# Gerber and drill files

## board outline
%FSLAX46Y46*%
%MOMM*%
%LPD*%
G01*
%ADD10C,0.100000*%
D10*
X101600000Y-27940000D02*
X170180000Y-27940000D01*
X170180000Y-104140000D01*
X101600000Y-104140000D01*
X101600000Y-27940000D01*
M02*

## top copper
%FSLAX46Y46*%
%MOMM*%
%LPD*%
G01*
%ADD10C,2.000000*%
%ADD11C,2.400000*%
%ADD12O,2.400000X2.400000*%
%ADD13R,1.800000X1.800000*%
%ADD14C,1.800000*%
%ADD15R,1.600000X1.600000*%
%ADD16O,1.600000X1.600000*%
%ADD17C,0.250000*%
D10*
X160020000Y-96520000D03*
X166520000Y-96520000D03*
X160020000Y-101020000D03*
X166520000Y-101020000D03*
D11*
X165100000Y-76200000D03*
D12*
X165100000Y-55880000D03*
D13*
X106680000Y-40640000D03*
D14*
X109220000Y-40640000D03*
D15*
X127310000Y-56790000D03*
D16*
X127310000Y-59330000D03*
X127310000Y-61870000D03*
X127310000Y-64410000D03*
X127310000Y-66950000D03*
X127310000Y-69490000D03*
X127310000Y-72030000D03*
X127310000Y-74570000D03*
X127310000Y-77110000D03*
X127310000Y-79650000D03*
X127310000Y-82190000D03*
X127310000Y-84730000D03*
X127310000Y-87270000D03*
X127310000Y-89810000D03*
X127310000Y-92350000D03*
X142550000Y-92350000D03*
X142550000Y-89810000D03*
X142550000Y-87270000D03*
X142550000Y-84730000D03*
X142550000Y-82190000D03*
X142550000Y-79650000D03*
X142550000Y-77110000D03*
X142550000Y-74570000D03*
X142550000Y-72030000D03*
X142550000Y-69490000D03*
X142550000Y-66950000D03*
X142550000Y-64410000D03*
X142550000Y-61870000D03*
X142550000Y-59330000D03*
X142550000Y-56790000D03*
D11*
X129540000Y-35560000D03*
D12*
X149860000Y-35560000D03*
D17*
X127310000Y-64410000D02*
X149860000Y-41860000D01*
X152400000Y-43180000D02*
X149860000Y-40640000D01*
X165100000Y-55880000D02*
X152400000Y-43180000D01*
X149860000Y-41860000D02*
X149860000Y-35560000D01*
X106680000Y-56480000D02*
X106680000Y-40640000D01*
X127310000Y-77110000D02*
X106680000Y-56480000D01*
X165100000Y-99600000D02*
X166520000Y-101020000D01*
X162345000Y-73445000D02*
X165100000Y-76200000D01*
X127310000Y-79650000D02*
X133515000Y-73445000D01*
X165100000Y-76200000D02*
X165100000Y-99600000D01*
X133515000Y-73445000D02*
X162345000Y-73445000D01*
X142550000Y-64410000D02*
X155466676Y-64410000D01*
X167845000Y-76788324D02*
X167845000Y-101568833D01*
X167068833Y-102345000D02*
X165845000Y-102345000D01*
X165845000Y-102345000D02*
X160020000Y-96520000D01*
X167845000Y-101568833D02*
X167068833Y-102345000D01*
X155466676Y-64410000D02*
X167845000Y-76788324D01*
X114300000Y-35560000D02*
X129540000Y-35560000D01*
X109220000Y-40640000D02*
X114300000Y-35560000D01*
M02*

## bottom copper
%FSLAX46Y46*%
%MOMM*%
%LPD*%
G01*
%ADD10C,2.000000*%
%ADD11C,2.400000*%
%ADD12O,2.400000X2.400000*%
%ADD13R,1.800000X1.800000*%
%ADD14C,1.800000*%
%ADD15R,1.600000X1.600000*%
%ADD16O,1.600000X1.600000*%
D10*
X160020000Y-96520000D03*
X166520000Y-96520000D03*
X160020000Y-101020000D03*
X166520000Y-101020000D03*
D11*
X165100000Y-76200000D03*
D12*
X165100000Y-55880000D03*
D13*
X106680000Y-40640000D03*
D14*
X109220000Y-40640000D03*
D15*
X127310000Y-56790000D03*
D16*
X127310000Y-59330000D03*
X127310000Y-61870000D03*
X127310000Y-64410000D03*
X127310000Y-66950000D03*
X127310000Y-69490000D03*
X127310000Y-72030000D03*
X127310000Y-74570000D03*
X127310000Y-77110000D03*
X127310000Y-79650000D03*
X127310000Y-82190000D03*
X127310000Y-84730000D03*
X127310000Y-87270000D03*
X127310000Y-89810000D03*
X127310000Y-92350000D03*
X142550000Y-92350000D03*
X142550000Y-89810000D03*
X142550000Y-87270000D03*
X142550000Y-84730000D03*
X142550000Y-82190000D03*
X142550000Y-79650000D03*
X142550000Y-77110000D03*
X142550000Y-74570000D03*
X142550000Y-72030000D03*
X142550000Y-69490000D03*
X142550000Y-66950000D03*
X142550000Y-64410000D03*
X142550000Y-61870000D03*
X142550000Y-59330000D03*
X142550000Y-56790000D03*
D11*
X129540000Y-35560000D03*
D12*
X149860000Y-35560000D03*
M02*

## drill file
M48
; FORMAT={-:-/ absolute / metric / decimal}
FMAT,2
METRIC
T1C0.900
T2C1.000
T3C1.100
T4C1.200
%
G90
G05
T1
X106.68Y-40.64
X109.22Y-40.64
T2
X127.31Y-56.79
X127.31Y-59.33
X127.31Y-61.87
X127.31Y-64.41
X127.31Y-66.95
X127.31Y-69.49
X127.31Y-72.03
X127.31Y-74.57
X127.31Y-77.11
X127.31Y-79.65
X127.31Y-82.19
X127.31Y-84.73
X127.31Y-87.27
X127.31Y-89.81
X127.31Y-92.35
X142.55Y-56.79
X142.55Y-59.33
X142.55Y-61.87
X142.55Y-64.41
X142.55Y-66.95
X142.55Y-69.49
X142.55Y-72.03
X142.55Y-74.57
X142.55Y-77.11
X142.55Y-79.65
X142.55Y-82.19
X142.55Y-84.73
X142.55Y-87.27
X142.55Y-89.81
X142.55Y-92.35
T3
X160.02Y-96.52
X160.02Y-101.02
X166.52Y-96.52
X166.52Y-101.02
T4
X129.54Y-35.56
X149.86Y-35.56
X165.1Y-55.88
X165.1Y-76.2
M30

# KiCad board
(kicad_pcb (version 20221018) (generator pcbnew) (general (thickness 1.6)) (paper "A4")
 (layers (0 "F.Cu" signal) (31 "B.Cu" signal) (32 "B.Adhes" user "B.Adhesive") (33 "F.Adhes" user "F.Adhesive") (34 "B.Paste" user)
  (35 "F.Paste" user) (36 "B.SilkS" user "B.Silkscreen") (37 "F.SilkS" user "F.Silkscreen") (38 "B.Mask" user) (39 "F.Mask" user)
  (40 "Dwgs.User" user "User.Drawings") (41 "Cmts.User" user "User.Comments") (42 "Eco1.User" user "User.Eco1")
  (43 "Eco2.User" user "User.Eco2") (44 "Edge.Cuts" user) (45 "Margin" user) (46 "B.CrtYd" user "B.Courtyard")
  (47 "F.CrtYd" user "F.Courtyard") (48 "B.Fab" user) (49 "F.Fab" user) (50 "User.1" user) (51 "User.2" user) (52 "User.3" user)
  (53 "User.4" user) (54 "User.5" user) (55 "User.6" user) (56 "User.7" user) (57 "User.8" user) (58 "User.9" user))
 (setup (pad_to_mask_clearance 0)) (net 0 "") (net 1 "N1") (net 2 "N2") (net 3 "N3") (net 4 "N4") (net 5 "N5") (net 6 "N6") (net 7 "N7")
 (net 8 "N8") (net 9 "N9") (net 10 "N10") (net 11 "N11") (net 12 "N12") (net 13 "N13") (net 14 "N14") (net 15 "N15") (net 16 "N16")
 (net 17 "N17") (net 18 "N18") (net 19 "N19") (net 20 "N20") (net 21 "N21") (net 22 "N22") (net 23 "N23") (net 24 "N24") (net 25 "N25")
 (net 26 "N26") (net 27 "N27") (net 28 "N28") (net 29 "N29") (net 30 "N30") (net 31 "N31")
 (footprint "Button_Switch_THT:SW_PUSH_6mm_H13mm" (layer "F.Cu") (at 160.02 96.52)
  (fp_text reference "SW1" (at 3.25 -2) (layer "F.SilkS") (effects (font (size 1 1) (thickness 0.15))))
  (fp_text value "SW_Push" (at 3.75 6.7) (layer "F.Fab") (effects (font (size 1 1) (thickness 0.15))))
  (pad "1" thru_hole circle (at 0 0 90) (size 2 2) (drill 1.1) (layers "*.Cu" "*.Mask") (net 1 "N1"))
  (pad "1" thru_hole circle (at 6.5 0 90) (size 2 2) (drill 1.1) (layers "*.Cu" "*.Mask") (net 1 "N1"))
  (pad "2" thru_hole circle (at 0 4.5 90) (size 2 2) (drill 1.1) (layers "*.Cu" "*.Mask") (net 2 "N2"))
  (pad "2" thru_hole circle (at 6.5 4.5 90) (size 2 2) (drill 1.1) (layers "*.Cu" "*.Mask") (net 2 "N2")))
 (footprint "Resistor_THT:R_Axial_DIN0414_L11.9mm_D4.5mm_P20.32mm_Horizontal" (layer "F.Cu") (at 165.1 76.2 90)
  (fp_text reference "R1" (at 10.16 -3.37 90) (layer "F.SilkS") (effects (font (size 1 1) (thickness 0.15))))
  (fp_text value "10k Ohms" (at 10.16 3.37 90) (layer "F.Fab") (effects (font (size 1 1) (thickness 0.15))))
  (pad "1" thru_hole circle (at 0 0 90) (size 2.4 2.4) (drill 1.2) (layers "*.Cu" "*.Mask") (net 2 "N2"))
  (pad "2" thru_hole oval (at 20.32 0 90) (size 2.4 2.4) (drill 1.2) (layers "*.Cu" "*.Mask") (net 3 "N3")))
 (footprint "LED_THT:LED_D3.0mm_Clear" (layer "F.Cu") (at 106.68 40.64)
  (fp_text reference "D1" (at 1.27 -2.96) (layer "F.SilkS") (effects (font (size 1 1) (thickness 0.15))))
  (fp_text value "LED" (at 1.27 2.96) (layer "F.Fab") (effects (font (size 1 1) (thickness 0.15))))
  (pad "1" thru_hole rect (at 0 0) (size 1.8 1.8) (drill 0.9) (layers "*.Cu" "*.Mask") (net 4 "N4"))
  (pad "2" thru_hole circle (at 2.54 0) (size 1.8 1.8) (drill 0.9) (layers "*.Cu" "*.Mask") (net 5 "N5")))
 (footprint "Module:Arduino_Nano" (layer "F.Cu") (at 127.31 56.79)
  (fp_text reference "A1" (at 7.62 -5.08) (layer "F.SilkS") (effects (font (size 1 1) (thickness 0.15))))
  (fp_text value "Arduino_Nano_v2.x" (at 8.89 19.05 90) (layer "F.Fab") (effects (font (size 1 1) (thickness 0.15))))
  (pad "1" thru_hole rect (at 0 0) (size 1.6 1.6) (drill 1) (layers "*.Cu" "*.Mask") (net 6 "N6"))
  (pad "2" thru_hole oval (at 0 2.54) (size 1.6 1.6) (drill 1) (layers "*.Cu" "*.Mask") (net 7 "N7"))
  (pad "3" thru_hole oval (at 0 5.08) (size 1.6 1.6) (drill 1) (layers "*.Cu" "*.Mask") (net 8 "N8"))
  (pad "4" thru_hole oval (at 0 7.62) (size 1.6 1.6) (drill 1) (layers "*.Cu" "*.Mask") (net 3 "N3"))
  (pad "5" thru_hole oval (at 0 10.16) (size 1.6 1.6) (drill 1) (layers "*.Cu" "*.Mask") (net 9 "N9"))
  (pad "6" thru_hole oval (at 0 12.7) (size 1.6 1.6) (drill 1) (layers "*.Cu" "*.Mask") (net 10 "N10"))
  (pad "7" thru_hole oval (at 0 15.24) (size 1.6 1.6) (drill 1) (layers "*.Cu" "*.Mask") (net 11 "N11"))
  (pad "8" thru_hole oval (at 0 17.78) (size 1.6 1.6) (drill 1) (layers "*.Cu" "*.Mask") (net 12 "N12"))
  (pad "9" thru_hole oval (at 0 20.32) (size 1.6 1.6) (drill 1) (layers "*.Cu" "*.Mask") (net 4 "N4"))
  (pad "10" thru_hole oval (at 0 22.86) (size 1.6 1.6) (drill 1) (layers "*.Cu" "*.Mask") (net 2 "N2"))
  (pad "11" thru_hole oval (at 0 25.4) (size 1.6 1.6) (drill 1) (layers "*.Cu" "*.Mask") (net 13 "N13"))
  (pad "12" thru_hole oval (at 0 27.94) (size 1.6 1.6) (drill 1) (layers "*.Cu" "*.Mask") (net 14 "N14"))
  (pad "13" thru_hole oval (at 0 30.48) (size 1.6 1.6) (drill 1) (layers "*.Cu" "*.Mask") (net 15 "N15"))
  (pad "14" thru_hole oval (at 0 33.02) (size 1.6 1.6) (drill 1) (layers "*.Cu" "*.Mask") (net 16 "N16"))
  (pad "15" thru_hole oval (at 0 35.56) (size 1.6 1.6) (drill 1) (layers "*.Cu" "*.Mask") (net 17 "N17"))
  (pad "16" thru_hole oval (at 15.24 35.56) (size 1.6 1.6) (drill 1) (layers "*.Cu" "*.Mask") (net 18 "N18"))
  (pad "17" thru_hole oval (at 15.24 33.02) (size 1.6 1.6) (drill 1) (layers "*.Cu" "*.Mask") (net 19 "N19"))
  (pad "18" thru_hole oval (at 15.24 30.48) (size 1.6 1.6) (drill 1) (layers "*.Cu" "*.Mask") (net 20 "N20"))
  (pad "19" thru_hole oval (at 15.24 27.94) (size 1.6 1.6) (drill 1) (layers "*.Cu" "*.Mask") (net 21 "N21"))
  (pad "20" thru_hole oval (at 15.24 25.4) (size 1.6 1.6) (drill 1) (layers "*.Cu" "*.Mask") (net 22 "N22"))
  (pad "21" thru_hole oval (at 15.24 22.86) (size 1.6 1.6) (drill 1) (layers "*.Cu" "*.Mask") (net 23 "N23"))
  (pad "22" thru_hole oval (at 15.24 20.32) (size 1.6 1.6) (drill 1) (layers "*.Cu" "*.Mask") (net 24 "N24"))
  (pad "23" thru_hole oval (at 15.24 17.78) (size 1.6 1.6) (drill 1) (layers "*.Cu" "*.Mask") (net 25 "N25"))
  (pad "24" thru_hole oval (at 15.24 15.24) (size 1.6 1.6) (drill 1) (layers "*.Cu" "*.Mask") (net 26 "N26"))
  (pad "25" thru_hole oval (at 15.24 12.7) (size 1.6 1.6) (drill 1) (layers "*.Cu" "*.Mask") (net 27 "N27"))
  (pad "26" thru_hole oval (at 15.24 10.16) (size 1.6 1.6) (drill 1) (layers "*.Cu" "*.Mask") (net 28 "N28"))
  (pad "27" thru_hole oval (at 15.24 7.62) (size 1.6 1.6) (drill 1) (layers "*.Cu" "*.Mask") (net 1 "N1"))
  (pad "28" thru_hole oval (at 15.24 5.08) (size 1.6 1.6) (drill 1) (layers "*.Cu" "*.Mask") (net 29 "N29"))
  (pad "29" thru_hole oval (at 15.24 2.54) (size 1.6 1.6) (drill 1) (layers "*.Cu" "*.Mask") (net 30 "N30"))
  (pad "30" thru_hole oval (at 15.24 0) (size 1.6 1.6) (drill 1) (layers "*.Cu" "*.Mask") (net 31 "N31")))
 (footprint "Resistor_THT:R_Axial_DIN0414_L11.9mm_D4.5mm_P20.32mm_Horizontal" (layer "F.Cu") (at 129.54 35.56)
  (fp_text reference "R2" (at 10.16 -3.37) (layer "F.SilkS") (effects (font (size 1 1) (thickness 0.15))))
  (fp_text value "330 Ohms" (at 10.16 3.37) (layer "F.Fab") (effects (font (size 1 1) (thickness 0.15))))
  (pad "1" thru_hole circle (at 0 0) (size 2.4 2.4) (drill 1.2) (layers "*.Cu" "*.Mask") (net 5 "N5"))
  (pad "2" thru_hole oval (at 20.32 0) (size 2.4 2.4) (drill 1.2) (layers "*.Cu" "*.Mask") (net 3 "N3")))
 (gr_rect (start 101.6 27.94) (end 170.18 104.14) (stroke (width 0.1) (type default)) (fill none) (layer "Edge.Cuts"))
 (segment (start 127.31 64.41) (end 149.86 41.86) (width 0.25) (layer "F.Cu") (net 3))
 (segment (start 152.4 43.18) (end 149.86 40.64) (width 0.25) (layer "F.Cu") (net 3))
 (segment (start 165.1 55.88) (end 152.4 43.18) (width 0.25) (layer "F.Cu") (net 3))
 (segment (start 149.86 41.86) (end 149.86 35.56) (width 0.25) (layer "F.Cu") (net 3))
 (segment (start 106.68 56.48) (end 106.68 40.64) (width 0.25) (layer "F.Cu") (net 4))
 (segment (start 127.31 77.11) (end 106.68 56.48) (width 0.25) (layer "F.Cu") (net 4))
 (segment (start 165.1 99.6) (end 166.52 101.02) (width 0.25) (layer "F.Cu") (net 2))
 (segment (start 162.345 73.445) (end 165.1 76.2) (width 0.25) (layer "F.Cu") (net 2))
 (segment (start 127.31 79.65) (end 133.515 73.445) (width 0.25) (layer "F.Cu") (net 2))
 (segment (start 165.1 76.2) (end 165.1 99.6) (width 0.25) (layer "F.Cu") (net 2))
 (segment (start 133.515 73.445) (end 162.345 73.445) (width 0.25) (layer "F.Cu") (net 2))
 (segment (start 142.55 64.41) (end 155.466676 64.41) (width 0.25) (layer "F.Cu") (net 1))
 (segment (start 167.845 76.788324) (end 167.845 101.568833) (width 0.25) (layer "F.Cu") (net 1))
 (segment (start 167.068833 102.345) (end 165.845 102.345) (width 0.25) (layer "F.Cu") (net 1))
 (segment (start 165.845 102.345) (end 160.02 96.52) (width 0.25) (layer "F.Cu") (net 1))
 (segment (start 167.845 101.568833) (end 167.068833 102.345) (width 0.25) (layer "F.Cu") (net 1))
 (segment (start 155.466676 64.41) (end 167.845 76.788324) (width 0.25) (layer "F.Cu") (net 1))
 (segment (start 114.3 35.56) (end 129.54 35.56) (width 0.25) (layer "F.Cu") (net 5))
 (segment (start 109.22 40.64) (end 114.3 35.56) (width 0.25) (layer "F.Cu") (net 5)))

